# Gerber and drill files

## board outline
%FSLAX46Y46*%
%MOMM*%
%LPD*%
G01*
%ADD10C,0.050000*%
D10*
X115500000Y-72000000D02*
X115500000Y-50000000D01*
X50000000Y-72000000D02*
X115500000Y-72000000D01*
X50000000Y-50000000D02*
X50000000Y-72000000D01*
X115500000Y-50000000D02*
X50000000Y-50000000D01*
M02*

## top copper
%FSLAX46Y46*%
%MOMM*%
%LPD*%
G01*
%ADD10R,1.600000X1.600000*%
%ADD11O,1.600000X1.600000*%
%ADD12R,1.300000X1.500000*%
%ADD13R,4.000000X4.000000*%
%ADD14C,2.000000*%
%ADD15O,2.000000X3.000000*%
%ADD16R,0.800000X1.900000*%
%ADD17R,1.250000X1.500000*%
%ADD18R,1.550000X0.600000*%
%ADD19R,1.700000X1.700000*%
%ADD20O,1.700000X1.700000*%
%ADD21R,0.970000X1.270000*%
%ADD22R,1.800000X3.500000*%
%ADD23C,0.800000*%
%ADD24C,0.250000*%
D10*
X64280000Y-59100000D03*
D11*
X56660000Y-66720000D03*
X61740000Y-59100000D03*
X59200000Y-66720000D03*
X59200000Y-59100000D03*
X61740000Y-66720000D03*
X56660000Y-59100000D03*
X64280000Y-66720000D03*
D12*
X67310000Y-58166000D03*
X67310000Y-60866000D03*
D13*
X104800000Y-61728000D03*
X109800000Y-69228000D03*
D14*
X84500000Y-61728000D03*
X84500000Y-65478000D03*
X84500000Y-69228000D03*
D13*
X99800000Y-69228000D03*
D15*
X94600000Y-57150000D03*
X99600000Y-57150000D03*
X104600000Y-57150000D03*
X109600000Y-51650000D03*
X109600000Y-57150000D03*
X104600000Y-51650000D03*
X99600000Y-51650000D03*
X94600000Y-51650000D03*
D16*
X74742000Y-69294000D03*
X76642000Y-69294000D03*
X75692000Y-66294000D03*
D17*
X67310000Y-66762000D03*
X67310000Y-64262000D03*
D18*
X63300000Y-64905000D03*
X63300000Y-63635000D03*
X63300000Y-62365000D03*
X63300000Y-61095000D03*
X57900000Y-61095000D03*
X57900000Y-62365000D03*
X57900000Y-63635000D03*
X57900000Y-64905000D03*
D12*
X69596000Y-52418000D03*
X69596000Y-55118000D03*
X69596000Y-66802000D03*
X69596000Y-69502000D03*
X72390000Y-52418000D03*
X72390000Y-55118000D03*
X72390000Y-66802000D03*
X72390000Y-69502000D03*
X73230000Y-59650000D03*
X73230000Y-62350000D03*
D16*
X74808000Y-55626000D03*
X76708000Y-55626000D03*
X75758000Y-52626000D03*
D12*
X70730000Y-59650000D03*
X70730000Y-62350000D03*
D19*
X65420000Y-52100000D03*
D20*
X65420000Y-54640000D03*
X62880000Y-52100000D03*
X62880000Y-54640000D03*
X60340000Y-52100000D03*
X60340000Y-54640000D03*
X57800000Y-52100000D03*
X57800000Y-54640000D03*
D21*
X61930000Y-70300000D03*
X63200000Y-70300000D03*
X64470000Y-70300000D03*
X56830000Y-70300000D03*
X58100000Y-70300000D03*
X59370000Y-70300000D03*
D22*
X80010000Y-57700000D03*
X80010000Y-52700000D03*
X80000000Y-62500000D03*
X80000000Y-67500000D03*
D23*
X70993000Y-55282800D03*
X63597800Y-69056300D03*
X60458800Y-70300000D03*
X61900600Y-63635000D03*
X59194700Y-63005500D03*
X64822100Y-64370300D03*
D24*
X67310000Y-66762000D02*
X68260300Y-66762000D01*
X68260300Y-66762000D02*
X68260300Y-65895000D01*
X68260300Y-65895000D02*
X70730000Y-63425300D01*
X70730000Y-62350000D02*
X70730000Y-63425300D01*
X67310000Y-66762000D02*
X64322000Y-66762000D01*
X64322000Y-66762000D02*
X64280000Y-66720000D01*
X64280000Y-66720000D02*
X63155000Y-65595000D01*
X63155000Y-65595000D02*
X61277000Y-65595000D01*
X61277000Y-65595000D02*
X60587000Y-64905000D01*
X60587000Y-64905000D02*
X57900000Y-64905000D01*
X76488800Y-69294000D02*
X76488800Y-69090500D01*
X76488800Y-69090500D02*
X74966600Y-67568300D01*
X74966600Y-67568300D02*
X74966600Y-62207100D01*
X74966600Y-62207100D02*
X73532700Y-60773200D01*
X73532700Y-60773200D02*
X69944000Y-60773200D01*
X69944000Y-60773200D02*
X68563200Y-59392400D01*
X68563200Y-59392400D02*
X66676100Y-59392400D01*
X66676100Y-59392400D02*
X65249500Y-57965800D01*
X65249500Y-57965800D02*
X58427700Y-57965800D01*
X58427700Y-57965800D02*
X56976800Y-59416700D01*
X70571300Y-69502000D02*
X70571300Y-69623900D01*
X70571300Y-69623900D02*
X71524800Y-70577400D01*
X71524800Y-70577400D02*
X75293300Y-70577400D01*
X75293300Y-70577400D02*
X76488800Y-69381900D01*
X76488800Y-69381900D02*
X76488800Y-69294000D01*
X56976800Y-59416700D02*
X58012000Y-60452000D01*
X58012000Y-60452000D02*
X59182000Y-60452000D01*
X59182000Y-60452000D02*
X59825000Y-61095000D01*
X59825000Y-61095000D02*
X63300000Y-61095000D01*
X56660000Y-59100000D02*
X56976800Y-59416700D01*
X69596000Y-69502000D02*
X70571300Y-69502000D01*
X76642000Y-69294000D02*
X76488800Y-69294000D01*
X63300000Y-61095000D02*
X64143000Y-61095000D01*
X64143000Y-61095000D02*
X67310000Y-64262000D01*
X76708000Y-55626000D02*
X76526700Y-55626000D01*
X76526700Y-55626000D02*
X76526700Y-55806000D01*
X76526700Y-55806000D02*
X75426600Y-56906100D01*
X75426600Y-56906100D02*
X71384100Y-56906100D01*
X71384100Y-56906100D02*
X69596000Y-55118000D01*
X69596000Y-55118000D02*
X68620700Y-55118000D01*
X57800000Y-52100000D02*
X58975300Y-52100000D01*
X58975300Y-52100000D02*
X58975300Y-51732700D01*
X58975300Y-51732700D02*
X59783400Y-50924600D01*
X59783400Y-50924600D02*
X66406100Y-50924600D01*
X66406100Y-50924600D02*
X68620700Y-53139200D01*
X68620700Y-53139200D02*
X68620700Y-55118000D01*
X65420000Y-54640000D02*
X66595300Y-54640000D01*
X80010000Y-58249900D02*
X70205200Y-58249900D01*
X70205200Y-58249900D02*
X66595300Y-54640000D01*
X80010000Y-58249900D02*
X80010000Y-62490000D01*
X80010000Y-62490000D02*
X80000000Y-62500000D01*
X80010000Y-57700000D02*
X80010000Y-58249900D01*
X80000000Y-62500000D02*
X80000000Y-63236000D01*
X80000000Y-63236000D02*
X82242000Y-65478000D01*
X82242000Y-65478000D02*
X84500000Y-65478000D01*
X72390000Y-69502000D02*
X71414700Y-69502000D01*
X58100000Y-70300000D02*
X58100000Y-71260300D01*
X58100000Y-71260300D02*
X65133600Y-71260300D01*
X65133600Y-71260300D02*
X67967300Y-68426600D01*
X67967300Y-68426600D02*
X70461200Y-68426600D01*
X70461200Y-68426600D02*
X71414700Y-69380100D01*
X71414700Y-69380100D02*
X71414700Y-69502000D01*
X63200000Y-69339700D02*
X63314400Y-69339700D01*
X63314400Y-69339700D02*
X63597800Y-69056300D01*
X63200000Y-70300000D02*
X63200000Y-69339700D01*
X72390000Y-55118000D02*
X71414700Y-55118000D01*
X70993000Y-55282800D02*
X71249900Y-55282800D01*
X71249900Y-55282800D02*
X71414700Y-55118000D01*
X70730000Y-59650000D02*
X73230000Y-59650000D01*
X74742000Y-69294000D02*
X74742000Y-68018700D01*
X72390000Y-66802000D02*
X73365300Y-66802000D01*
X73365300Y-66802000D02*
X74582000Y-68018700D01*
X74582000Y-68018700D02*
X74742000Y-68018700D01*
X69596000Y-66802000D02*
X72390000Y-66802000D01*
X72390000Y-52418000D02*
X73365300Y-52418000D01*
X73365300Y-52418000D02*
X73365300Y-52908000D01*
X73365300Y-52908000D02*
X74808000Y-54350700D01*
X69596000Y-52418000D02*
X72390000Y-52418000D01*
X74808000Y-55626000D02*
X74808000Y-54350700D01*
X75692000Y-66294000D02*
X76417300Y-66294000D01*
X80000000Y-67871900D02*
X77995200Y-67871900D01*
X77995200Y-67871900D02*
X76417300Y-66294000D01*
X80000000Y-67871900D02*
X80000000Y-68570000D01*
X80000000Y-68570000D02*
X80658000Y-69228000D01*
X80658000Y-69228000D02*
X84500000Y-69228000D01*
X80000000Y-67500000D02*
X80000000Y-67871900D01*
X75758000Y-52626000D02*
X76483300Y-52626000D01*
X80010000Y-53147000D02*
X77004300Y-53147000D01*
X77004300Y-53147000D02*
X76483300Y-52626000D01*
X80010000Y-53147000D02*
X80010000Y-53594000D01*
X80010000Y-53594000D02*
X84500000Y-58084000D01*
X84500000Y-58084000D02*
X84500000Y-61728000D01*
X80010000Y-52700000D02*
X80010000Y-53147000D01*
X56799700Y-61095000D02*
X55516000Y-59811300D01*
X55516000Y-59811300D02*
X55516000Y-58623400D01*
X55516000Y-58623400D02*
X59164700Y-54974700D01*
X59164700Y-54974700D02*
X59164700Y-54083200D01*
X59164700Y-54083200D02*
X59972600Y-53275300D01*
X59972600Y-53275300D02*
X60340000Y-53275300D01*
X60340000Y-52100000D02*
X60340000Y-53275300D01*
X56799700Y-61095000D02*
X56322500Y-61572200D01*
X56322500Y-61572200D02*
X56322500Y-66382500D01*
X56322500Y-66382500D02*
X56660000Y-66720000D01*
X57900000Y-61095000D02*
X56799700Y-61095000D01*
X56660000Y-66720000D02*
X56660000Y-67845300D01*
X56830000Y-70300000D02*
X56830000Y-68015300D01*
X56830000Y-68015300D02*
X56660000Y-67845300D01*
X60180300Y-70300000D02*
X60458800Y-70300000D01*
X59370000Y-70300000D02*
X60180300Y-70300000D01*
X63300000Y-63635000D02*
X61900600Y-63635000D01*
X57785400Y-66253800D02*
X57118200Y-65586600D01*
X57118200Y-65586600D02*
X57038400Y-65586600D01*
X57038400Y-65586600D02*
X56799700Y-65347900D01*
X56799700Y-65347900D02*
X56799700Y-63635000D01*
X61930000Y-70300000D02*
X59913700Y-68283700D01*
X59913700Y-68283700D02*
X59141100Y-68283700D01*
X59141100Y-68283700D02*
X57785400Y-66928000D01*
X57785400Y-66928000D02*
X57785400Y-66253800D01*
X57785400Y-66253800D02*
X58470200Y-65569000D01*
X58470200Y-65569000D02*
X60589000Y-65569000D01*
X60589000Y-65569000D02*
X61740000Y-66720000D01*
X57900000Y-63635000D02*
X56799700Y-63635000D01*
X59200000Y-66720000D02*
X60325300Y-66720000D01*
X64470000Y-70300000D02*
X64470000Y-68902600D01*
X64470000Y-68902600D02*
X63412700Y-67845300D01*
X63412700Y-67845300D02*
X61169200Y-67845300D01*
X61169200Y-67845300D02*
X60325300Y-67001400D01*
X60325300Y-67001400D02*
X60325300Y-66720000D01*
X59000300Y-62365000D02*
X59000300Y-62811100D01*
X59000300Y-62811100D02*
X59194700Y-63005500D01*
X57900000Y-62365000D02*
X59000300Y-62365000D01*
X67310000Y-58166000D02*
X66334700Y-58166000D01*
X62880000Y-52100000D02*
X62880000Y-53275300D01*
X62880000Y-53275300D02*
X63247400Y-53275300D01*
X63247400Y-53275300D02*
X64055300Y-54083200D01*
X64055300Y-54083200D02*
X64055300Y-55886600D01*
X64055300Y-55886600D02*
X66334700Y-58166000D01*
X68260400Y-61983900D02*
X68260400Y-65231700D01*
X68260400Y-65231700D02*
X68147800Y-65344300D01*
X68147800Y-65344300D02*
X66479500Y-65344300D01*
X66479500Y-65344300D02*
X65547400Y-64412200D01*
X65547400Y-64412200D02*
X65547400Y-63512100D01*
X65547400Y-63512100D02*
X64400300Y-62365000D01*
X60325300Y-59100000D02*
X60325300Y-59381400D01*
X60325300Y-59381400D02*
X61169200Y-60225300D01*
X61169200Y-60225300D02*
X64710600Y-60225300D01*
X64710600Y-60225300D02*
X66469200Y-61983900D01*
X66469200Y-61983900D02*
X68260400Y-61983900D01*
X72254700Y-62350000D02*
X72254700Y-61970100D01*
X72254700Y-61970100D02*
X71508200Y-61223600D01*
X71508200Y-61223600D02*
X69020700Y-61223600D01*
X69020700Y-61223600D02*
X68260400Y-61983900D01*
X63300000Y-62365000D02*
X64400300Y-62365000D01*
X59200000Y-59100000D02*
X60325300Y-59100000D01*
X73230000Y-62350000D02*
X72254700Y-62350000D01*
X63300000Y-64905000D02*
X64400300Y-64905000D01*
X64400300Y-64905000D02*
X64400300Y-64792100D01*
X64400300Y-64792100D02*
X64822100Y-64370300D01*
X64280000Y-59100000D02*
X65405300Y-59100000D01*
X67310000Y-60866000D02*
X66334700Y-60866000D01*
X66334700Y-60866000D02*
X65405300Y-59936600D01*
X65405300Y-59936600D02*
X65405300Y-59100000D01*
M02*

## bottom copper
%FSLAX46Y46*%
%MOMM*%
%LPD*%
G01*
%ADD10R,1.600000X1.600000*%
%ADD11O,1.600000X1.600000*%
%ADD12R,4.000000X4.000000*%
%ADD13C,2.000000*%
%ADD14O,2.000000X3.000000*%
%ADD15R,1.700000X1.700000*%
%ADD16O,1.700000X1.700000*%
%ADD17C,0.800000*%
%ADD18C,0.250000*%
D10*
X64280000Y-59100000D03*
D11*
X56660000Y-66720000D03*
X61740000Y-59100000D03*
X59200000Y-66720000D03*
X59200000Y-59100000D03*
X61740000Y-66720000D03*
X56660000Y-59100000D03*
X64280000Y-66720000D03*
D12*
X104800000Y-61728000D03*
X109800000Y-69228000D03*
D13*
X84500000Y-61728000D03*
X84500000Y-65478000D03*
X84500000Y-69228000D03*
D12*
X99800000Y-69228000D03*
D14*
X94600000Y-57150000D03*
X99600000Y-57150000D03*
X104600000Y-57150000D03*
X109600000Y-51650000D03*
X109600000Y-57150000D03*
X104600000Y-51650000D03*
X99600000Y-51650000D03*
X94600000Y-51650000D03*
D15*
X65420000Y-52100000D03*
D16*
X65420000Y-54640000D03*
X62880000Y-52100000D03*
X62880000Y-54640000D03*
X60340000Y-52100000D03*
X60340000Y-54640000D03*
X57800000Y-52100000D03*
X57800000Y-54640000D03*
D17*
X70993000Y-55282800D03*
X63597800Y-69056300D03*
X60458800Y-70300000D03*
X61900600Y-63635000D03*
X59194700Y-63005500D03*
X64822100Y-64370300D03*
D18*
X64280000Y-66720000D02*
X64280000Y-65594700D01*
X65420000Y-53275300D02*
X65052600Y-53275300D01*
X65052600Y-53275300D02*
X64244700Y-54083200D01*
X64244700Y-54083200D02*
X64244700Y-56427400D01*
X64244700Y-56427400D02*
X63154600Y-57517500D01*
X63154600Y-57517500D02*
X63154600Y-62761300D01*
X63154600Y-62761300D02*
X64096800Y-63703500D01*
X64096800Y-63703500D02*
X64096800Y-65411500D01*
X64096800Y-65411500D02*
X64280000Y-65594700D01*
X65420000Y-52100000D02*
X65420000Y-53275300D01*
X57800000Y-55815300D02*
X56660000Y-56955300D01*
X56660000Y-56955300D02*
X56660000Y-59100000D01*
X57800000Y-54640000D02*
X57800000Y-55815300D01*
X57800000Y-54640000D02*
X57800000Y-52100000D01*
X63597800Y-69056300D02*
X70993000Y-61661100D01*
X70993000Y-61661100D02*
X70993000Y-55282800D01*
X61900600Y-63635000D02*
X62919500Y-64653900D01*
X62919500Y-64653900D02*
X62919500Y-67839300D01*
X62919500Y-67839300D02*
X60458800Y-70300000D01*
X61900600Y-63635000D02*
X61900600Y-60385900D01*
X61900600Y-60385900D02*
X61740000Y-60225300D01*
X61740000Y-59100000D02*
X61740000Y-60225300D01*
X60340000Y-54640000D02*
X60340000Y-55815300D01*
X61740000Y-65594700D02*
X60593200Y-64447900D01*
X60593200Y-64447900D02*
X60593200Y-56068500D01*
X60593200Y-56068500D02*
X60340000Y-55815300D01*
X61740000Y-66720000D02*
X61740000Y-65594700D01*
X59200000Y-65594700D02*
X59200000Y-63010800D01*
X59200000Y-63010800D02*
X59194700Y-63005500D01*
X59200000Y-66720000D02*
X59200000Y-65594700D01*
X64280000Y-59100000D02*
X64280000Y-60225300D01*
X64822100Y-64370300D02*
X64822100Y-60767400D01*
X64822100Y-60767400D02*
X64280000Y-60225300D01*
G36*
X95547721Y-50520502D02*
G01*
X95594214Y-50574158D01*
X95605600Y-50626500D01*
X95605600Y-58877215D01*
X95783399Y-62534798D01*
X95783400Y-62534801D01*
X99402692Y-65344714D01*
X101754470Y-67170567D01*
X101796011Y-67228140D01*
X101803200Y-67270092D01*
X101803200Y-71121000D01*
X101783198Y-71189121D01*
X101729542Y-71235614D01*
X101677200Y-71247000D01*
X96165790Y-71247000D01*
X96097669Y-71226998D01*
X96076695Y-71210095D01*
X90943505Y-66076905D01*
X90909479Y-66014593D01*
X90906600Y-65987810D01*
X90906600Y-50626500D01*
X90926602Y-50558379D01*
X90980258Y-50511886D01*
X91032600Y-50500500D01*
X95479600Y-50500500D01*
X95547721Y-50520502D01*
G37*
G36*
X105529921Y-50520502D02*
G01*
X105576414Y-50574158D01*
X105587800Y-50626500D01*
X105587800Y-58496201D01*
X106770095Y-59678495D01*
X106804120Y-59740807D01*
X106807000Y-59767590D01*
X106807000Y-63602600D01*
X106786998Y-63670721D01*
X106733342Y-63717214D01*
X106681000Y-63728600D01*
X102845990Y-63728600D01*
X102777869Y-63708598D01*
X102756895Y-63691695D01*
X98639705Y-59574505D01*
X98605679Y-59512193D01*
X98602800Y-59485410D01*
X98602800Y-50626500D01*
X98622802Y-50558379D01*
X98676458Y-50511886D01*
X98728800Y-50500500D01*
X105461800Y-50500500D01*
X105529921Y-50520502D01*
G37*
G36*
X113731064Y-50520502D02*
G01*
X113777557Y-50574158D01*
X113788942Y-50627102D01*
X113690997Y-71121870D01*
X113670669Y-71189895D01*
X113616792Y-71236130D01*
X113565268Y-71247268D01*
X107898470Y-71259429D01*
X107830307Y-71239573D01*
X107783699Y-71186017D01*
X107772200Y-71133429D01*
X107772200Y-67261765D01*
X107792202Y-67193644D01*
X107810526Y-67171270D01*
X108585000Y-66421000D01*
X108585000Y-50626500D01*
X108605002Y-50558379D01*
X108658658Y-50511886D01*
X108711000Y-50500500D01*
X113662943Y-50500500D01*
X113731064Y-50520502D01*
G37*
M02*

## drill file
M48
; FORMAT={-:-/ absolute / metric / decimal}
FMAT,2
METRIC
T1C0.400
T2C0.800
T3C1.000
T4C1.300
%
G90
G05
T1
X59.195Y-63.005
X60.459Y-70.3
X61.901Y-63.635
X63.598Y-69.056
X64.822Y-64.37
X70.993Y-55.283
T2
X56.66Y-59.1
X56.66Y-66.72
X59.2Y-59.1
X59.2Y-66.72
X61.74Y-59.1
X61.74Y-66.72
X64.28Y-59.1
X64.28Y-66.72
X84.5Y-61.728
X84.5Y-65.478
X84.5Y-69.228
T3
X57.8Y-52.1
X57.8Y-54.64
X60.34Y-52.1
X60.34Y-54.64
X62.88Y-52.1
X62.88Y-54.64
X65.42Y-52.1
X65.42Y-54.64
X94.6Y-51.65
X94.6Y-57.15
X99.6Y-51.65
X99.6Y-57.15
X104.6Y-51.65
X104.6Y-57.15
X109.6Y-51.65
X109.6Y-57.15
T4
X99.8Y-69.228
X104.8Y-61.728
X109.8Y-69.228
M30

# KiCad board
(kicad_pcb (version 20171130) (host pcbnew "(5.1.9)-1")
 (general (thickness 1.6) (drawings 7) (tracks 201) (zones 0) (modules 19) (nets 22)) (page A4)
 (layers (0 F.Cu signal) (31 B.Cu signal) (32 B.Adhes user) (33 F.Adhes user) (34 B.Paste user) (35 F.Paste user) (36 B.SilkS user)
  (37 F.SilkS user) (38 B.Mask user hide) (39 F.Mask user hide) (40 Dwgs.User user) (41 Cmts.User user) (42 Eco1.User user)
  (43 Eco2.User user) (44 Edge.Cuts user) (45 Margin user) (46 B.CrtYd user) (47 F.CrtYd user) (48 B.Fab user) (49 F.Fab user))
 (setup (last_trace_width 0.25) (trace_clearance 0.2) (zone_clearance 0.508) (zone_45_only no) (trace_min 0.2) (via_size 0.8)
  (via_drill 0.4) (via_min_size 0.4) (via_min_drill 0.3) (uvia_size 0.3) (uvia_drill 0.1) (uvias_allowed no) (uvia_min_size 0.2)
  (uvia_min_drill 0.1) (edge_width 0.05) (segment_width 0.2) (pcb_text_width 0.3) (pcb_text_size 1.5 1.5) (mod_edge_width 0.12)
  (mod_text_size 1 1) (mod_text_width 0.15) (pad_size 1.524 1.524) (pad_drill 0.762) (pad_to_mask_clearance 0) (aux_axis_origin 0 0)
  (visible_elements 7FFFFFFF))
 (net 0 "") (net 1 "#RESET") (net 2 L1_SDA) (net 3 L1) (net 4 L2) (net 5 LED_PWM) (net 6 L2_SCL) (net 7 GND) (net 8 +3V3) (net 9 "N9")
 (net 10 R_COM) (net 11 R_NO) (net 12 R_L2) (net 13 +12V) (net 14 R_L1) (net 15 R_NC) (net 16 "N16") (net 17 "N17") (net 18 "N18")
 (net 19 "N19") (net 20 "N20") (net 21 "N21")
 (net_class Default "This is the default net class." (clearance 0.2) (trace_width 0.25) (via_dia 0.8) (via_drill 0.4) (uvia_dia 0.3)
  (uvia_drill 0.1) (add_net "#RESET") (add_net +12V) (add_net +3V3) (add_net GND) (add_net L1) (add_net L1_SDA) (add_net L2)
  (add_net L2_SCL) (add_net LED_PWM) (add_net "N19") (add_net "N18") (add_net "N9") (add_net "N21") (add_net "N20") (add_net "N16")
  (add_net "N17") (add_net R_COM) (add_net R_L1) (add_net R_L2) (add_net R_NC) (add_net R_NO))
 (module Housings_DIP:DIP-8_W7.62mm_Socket (layer F.Cu) (at 64.28 59.1 270)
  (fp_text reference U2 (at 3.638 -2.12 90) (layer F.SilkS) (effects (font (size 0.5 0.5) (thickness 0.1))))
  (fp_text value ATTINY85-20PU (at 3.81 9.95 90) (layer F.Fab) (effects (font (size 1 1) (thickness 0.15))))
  (pad 1 thru_hole rect (at 0 0 270) (size 1.6 1.6) (drill 0.8) (layers *.Cu *.Mask) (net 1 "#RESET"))
  (pad 5 thru_hole oval (at 7.62 7.62 270) (size 1.6 1.6) (drill 0.8) (layers *.Cu *.Mask) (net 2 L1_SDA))
  (pad 2 thru_hole oval (at 0 2.54 270) (size 1.6 1.6) (drill 0.8) (layers *.Cu *.Mask) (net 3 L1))
  (pad 6 thru_hole oval (at 7.62 5.08 270) (size 1.6 1.6) (drill 0.8) (layers *.Cu *.Mask) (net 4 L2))
  (pad 3 thru_hole oval (at 0 5.08 270) (size 1.6 1.6) (drill 0.8) (layers *.Cu *.Mask) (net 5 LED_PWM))
  (pad 7 thru_hole oval (at 7.62 2.54 270) (size 1.6 1.6) (drill 0.8) (layers *.Cu *.Mask) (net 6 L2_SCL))
  (pad 4 thru_hole oval (at 0 7.62 270) (size 1.6 1.6) (drill 0.8) (layers *.Cu *.Mask) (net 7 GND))
  (pad 8 thru_hole oval (at 7.62 0 270) (size 1.6 1.6) (drill 0.8) (layers *.Cu *.Mask) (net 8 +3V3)))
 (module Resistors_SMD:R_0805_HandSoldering (layer F.Cu) (at 67.31 59.516 270)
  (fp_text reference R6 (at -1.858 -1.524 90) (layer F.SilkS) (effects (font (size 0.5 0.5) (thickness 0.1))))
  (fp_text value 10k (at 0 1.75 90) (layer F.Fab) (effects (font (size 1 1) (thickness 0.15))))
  (pad 1 smd rect (at -1.35 0 270) (size 1.5 1.3) (layers F.Cu F.Paste F.Mask) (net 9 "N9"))
  (pad 2 smd rect (at 1.35 0 270) (size 1.5 1.3) (layers F.Cu F.Paste F.Mask) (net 1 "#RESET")))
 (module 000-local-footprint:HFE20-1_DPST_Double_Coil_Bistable (layer F.Cu) (at 84.5 65.478)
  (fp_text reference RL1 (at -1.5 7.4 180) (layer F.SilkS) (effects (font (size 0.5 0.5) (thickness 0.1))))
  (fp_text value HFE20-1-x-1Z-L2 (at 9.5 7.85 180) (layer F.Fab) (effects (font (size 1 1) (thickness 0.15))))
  (pad 3 thru_hole rect (at 20.3 -3.75) (size 4 4) (drill 1.3) (layers *.Cu *.Mask) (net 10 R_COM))
  (pad 4 thru_hole rect (at 25.3 3.75) (size 4 4) (drill 1.3) (layers *.Cu *.Mask) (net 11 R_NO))
  (pad 2 thru_hole circle (at 0 -3.75) (size 2 2) (drill 0.8) (layers *.Cu *.Mask) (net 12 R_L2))
  (pad 5 thru_hole circle (at 0 0) (size 2 2) (drill 0.8) (layers *.Cu *.Mask) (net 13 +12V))
  (pad 1 thru_hole circle (at 0 3.75) (size 2 2) (drill 0.8) (layers *.Cu *.Mask) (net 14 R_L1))
  (pad 6 thru_hole rect (at 15.3 3.75) (size 4 4) (drill 1.3) (layers *.Cu *.Mask) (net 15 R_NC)))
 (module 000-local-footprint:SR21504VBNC (layer F.Cu) (at 109.6 57.15 180)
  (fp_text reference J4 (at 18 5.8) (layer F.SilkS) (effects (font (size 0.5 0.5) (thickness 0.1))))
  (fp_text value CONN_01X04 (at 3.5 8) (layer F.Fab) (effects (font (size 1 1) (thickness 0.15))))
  (pad 4 thru_hole oval (at 15 0 180) (size 2 3) (drill 1) (layers *.Cu *.Mask) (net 15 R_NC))
  (pad 3 thru_hole oval (at 10 0 180) (size 2 3) (drill 1) (layers *.Cu *.Mask) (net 10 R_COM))
  (pad 2 thru_hole oval (at 5 0 180) (size 2 3) (drill 1) (layers *.Cu *.Mask) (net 10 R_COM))
  (pad 1 thru_hole oval (at 0 5.5 180) (size 2 3) (drill 1) (layers *.Cu *.Mask) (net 11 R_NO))
  (pad 1 thru_hole oval (at 0 0 180) (size 2 3) (drill 1) (layers *.Cu *.Mask) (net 11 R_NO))
  (pad 2 thru_hole oval (at 5 5.5 180) (size 2 3) (drill 1) (layers *.Cu *.Mask) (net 10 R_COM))
  (pad 3 thru_hole oval (at 10 5.5 180) (size 2 3) (drill 1) (layers *.Cu *.Mask) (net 10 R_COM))
  (pad 4 thru_hole oval (at 15 5.5 180) (size 2 3) (drill 1) (layers *.Cu *.Mask) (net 15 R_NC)))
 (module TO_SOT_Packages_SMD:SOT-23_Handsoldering (layer F.Cu) (at 75.692 67.794 90)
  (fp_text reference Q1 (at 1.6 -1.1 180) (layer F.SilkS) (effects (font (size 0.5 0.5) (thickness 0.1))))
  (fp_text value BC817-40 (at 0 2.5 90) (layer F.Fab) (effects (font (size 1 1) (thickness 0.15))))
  (pad 1 smd rect (at -1.5 -0.95 90) (size 1.9 0.8) (layers F.Cu F.Paste F.Mask) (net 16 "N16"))
  (pad 2 smd rect (at -1.5 0.95 90) (size 1.9 0.8) (layers F.Cu F.Paste F.Mask) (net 7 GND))
  (pad 3 smd rect (at 1.5 0 90) (size 1.9 0.8) (layers F.Cu F.Paste F.Mask) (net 14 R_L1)))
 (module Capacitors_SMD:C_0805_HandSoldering (layer F.Cu) (at 67.31 65.512 90)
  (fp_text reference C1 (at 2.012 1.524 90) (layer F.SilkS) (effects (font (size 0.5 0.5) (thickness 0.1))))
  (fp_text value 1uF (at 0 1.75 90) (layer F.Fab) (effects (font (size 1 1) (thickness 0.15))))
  (pad 1 smd rect (at -1.25 0 90) (size 1.5 1.25) (layers F.Cu F.Paste F.Mask) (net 8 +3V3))
  (pad 2 smd rect (at 1.25 0 90) (size 1.5 1.25) (layers F.Cu F.Paste F.Mask) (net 7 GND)))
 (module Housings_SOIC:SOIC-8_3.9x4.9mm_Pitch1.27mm (layer F.Cu) (at 60.6 63 180)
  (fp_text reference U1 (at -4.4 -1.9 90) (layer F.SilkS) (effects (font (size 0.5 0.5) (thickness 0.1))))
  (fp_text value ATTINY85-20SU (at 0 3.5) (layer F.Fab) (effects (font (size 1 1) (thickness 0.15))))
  (pad 1 smd rect (at -2.7 -1.905 180) (size 1.55 0.6) (layers F.Cu F.Paste F.Mask) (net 1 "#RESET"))
  (pad 2 smd rect (at -2.7 -0.635 180) (size 1.55 0.6) (layers F.Cu F.Paste F.Mask) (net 3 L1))
  (pad 3 smd rect (at -2.7 0.635 180) (size 1.55 0.6) (layers F.Cu F.Paste F.Mask) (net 5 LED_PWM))
  (pad 4 smd rect (at -2.7 1.905 180) (size 1.55 0.6) (layers F.Cu F.Paste F.Mask) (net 7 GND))
  (pad 5 smd rect (at 2.7 1.905 180) (size 1.55 0.6) (layers F.Cu F.Paste F.Mask) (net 2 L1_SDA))
  (pad 6 smd rect (at 2.7 0.635 180) (size 1.55 0.6) (layers F.Cu F.Paste F.Mask) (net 4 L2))
  (pad 7 smd rect (at 2.7 -0.635 180) (size 1.55 0.6) (layers F.Cu F.Paste F.Mask) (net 6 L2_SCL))
  (pad 8 smd rect (at 2.7 -1.905 180) (size 1.55 0.6) (layers F.Cu F.Paste F.Mask) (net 8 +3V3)))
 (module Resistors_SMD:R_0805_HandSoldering (layer F.Cu) (at 69.596 53.768 270)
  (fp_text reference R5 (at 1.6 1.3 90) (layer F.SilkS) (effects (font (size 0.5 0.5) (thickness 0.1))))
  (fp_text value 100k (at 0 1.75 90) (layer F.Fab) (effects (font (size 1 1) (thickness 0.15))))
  (pad 1 smd rect (at -1.35 0 270) (size 1.5 1.3) (layers F.Cu F.Paste F.Mask) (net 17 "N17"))
  (pad 2 smd rect (at 1.35 0 270) (size 1.5 1.3) (layers F.Cu F.Paste F.Mask) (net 7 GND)))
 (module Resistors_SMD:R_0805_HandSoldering (layer F.Cu) (at 69.596 68.152 270)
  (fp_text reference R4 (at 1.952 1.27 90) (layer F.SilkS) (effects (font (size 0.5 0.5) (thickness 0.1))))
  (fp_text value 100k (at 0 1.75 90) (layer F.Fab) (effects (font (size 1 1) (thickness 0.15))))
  (pad 1 smd rect (at -1.35 0 270) (size 1.5 1.3) (layers F.Cu F.Paste F.Mask) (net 16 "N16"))
  (pad 2 smd rect (at 1.35 0 270) (size 1.5 1.3) (layers F.Cu F.Paste F.Mask) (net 7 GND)))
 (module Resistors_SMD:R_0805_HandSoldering (layer F.Cu) (at 72.39 53.768 270)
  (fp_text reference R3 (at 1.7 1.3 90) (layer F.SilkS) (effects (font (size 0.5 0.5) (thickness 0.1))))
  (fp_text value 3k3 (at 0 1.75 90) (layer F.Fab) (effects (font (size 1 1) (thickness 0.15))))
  (pad 1 smd rect (at -1.35 0 270) (size 1.5 1.3) (layers F.Cu F.Paste F.Mask) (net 17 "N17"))
  (pad 2 smd rect (at 1.35 0 270) (size 1.5 1.3) (layers F.Cu F.Paste F.Mask) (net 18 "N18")))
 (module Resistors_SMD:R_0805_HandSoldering (layer F.Cu) (at 72.39 68.152 270)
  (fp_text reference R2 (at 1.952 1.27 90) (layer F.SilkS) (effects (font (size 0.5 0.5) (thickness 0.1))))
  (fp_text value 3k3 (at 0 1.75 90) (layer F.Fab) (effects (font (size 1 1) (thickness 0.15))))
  (pad 1 smd rect (at -1.35 0 270) (size 1.5 1.3) (layers F.Cu F.Paste F.Mask) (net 16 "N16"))
  (pad 2 smd rect (at 1.35 0 270) (size 1.5 1.3) (layers F.Cu F.Paste F.Mask) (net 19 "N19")))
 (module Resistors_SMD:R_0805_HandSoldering (layer F.Cu) (at 73.23 61 270)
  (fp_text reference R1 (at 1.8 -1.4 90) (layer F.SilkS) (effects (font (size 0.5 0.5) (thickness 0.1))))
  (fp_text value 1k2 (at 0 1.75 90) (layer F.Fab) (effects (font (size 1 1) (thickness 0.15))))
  (pad 1 smd rect (at -1.35 0 270) (size 1.5 1.3) (layers F.Cu F.Paste F.Mask) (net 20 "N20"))
  (pad 2 smd rect (at 1.35 0 270) (size 1.5 1.3) (layers F.Cu F.Paste F.Mask) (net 5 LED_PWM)))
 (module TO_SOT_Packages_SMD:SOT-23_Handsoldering (layer F.Cu) (at 75.758 54.126 90)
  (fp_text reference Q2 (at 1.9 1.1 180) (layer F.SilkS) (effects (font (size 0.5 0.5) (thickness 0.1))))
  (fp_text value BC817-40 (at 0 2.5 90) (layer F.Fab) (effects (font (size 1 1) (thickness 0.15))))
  (pad 1 smd rect (at -1.5 -0.95 90) (size 1.9 0.8) (layers F.Cu F.Paste F.Mask) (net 17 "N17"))
  (pad 2 smd rect (at -1.5 0.95 90) (size 1.9 0.8) (layers F.Cu F.Paste F.Mask) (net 7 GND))
  (pad 3 smd rect (at 1.5 0 90) (size 1.9 0.8) (layers F.Cu F.Paste F.Mask) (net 12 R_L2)))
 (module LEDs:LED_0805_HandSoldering (layer F.Cu) (at 70.73 61 270)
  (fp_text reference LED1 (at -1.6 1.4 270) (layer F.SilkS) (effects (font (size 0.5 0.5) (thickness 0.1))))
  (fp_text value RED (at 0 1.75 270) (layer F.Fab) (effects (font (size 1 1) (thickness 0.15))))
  (pad 1 smd rect (at -1.35 0 270) (size 1.5 1.3) (layers F.Cu F.Paste F.Mask) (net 20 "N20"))
  (pad 2 smd rect (at 1.35 0 270) (size 1.5 1.3) (layers F.Cu F.Paste F.Mask) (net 8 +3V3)))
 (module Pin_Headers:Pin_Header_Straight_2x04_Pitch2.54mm (layer F.Cu) (at 65.42 52.1 270)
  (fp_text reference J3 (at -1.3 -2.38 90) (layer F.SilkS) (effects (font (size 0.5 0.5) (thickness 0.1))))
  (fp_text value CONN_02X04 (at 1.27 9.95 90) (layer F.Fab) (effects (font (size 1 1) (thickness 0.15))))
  (pad 1 thru_hole rect (at 0 0 270) (size 1.7 1.7) (drill 1) (layers *.Cu *.Mask) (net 8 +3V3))
  (pad 2 thru_hole oval (at 2.54 0 270) (size 1.7 1.7) (drill 1) (layers *.Cu *.Mask) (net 13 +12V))
  (pad 3 thru_hole oval (at 0 2.54 270) (size 1.7 1.7) (drill 1) (layers *.Cu *.Mask) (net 9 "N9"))
  (pad 4 thru_hole oval (at 2.54 2.54 270) (size 1.7 1.7) (drill 1) (layers *.Cu *.Mask) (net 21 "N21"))
  (pad 5 thru_hole oval (at 0 5.08 270) (size 1.7 1.7) (drill 1) (layers *.Cu *.Mask) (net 2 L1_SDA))
  (pad 6 thru_hole oval (at 2.54 5.08 270) (size 1.7 1.7) (drill 1) (layers *.Cu *.Mask) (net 6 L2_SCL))
  (pad 7 thru_hole oval (at 0 7.62 270) (size 1.7 1.7) (drill 1) (layers *.Cu *.Mask) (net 7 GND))
  (pad 8 thru_hole oval (at 2.54 7.62 270) (size 1.7 1.7) (drill 1) (layers *.Cu *.Mask) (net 7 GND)))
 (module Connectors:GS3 (layer F.Cu) (at 63.2 70.3 90)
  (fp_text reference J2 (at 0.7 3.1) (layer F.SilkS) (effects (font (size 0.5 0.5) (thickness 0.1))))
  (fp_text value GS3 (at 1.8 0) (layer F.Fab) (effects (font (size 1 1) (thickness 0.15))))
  (pad 1 smd rect (at 0 -1.27 90) (size 1.27 0.97) (layers F.Cu F.Paste F.Mask) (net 6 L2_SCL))
  (pad 2 smd rect (at 0 0 90) (size 1.27 0.97) (layers F.Cu F.Paste F.Mask) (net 18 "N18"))
  (pad 3 smd rect (at 0 1.27 90) (size 1.27 0.97) (layers F.Cu F.Paste F.Mask) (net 4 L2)))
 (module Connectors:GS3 (layer F.Cu) (at 58.1 70.3 90)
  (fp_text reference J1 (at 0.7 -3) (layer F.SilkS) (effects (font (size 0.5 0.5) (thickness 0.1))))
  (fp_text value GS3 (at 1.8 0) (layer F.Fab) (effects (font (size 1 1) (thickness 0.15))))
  (pad 1 smd rect (at 0 -1.27 90) (size 1.27 0.97) (layers F.Cu F.Paste F.Mask) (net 2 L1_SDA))
  (pad 2 smd rect (at 0 0 90) (size 1.27 0.97) (layers F.Cu F.Paste F.Mask) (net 19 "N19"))
  (pad 3 smd rect (at 0 1.27 90) (size 1.27 0.97) (layers F.Cu F.Paste F.Mask) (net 3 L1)))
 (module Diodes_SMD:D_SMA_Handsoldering (layer F.Cu) (at 80.01 55.2 90)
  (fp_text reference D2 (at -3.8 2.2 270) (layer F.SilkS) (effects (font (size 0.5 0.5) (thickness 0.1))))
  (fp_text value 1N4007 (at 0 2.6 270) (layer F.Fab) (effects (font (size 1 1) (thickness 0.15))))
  (pad 1 smd rect (at -2.5 0 90) (size 3.5 1.8) (layers F.Cu F.Paste F.Mask) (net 13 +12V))
  (pad 2 smd rect (at 2.5 0 90) (size 3.5 1.8) (layers F.Cu F.Paste F.Mask) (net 12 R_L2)))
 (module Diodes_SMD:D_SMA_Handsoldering (layer F.Cu) (at 80 65 270)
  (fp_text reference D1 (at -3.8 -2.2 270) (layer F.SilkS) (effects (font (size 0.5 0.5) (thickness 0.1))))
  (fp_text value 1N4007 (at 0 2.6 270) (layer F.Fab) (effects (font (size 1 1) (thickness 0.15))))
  (pad 1 smd rect (at -2.5 0 270) (size 3.5 1.8) (layers F.Cu F.Paste F.Mask) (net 13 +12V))
  (pad 2 smd rect (at 2.5 0 270) (size 3.5 1.8) (layers F.Cu F.Paste F.Mask) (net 14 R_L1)))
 (gr_line (start 115.5 72) (end 115.5 50) (layer Edge.Cuts) (width 0.05))
 (gr_line (start 50 72) (end 115.5 72) (layer Edge.Cuts) (width 0.05))
 (gr_line (start 50 50) (end 50 72) (layer Edge.Cuts) (width 0.05))
 (gr_line (start 115.5 50) (end 50 50) (layer Edge.Cuts) (width 0.05))
 (segment (start 64.28 66.72) (end 64.28 65.5947) (width 0.25) (layer B.Cu) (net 8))
 (segment (start 65.42 53.2753) (end 65.0526 53.2753) (width 0.25) (layer B.Cu) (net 8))
 (segment (start 65.0526 53.2753) (end 64.2447 54.0832) (width 0.25) (layer B.Cu) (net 8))
 (segment (start 64.2447 54.0832) (end 64.2447 56.4274) (width 0.25) (layer B.Cu) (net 8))
 (segment (start 64.2447 56.4274) (end 63.1546 57.5175) (width 0.25) (layer B.Cu) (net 8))
 (segment (start 63.1546 57.5175) (end 63.1546 62.7613) (width 0.25) (layer B.Cu) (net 8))
 (segment (start 63.1546 62.7613) (end 64.0968 63.7035) (width 0.25) (layer B.Cu) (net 8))
 (segment (start 64.0968 63.7035) (end 64.0968 65.4115) (width 0.25) (layer B.Cu) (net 8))
 (segment (start 64.0968 65.4115) (end 64.28 65.5947) (width 0.25) (layer B.Cu) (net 8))
 (segment (start 67.31 66.762) (end 68.2603 66.762) (width 0.25) (layer F.Cu) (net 8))
 (segment (start 68.2603 66.762) (end 68.2603 65.895) (width 0.25) (layer F.Cu) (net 8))
 (segment (start 68.2603 65.895) (end 70.73 63.4253) (width 0.25) (layer F.Cu) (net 8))
 (segment (start 70.73 62.35) (end 70.73 63.4253) (width 0.25) (layer F.Cu) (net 8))
 (segment (start 67.31 66.762) (end 64.322 66.762) (width 0.25) (layer F.Cu) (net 8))
 (segment (start 64.322 66.762) (end 64.28 66.72) (width 0.25) (layer F.Cu) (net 8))
 (segment (start 65.42 52.1) (end 65.42 53.2753) (width 0.25) (layer B.Cu) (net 8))
 (segment (start 64.28 66.72) (end 63.155 65.595) (width 0.25) (layer F.Cu) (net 8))
 (segment (start 63.155 65.595) (end 61.277 65.595) (width 0.25) (layer F.Cu) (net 8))
 (segment (start 61.277 65.595) (end 60.587 64.905) (width 0.25) (layer F.Cu) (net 8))
 (segment (start 60.587 64.905) (end 57.9 64.905) (width 0.25) (layer F.Cu) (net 8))
 (segment (start 76.4888 69.294) (end 76.4888 69.0905) (width 0.25) (layer F.Cu) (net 7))
 (segment (start 76.4888 69.0905) (end 74.9666 67.5683) (width 0.25) (layer F.Cu) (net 7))
 (segment (start 74.9666 67.5683) (end 74.9666 62.2071) (width 0.25) (layer F.Cu) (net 7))
 (segment (start 74.9666 62.2071) (end 73.5327 60.7732) (width 0.25) (layer F.Cu) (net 7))
 (segment (start 73.5327 60.7732) (end 69.944 60.7732) (width 0.25) (layer F.Cu) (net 7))
 (segment (start 69.944 60.7732) (end 68.5632 59.3924) (width 0.25) (layer F.Cu) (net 7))
 (segment (start 68.5632 59.3924) (end 66.6761 59.3924) (width 0.25) (layer F.Cu) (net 7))
 (segment (start 66.6761 59.3924) (end 65.2495 57.9658) (width 0.25) (layer F.Cu) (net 7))
 (segment (start 65.2495 57.9658) (end 58.4277 57.9658) (width 0.25) (layer F.Cu) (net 7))
 (segment (start 58.4277 57.9658) (end 56.9768 59.4167) (width 0.25) (layer F.Cu) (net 7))
 (segment (start 70.5713 69.502) (end 70.5713 69.6239) (width 0.25) (layer F.Cu) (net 7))
 (segment (start 70.5713 69.6239) (end 71.5248 70.5774) (width 0.25) (layer F.Cu) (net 7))
 (segment (start 71.5248 70.5774) (end 75.2933 70.5774) (width 0.25) (layer F.Cu) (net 7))
 (segment (start 75.2933 70.5774) (end 76.4888 69.3819) (width 0.25) (layer F.Cu) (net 7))
 (segment (start 76.4888 69.3819) (end 76.4888 69.294) (width 0.25) (layer F.Cu) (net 7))
 (segment (start 56.9768 59.4167) (end 58.012 60.452) (width 0.25) (layer F.Cu) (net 7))
 (segment (start 58.012 60.452) (end 59.182 60.452) (width 0.25) (layer F.Cu) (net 7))
 (segment (start 59.182 60.452) (end 59.825 61.095) (width 0.25) (layer F.Cu) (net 7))
 (segment (start 59.825 61.095) (end 63.3 61.095) (width 0.25) (layer F.Cu) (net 7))
 (segment (start 56.66 59.1) (end 56.9768 59.4167) (width 0.25) (layer F.Cu) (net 7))
 (segment (start 69.596 69.502) (end 70.5713 69.502) (width 0.25) (layer F.Cu) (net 7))
 (segment (start 76.642 69.294) (end 76.4888 69.294) (width 0.25) (layer F.Cu) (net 7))
 (segment (start 63.3 61.095) (end 64.143 61.095) (width 0.25) (layer F.Cu) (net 7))
 (segment (start 64.143 61.095) (end 67.31 64.262) (width 0.25) (layer F.Cu) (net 7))
 (segment (start 76.708 55.626) (end 76.5267 55.626) (width 0.25) (layer F.Cu) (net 7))
 (segment (start 76.5267 55.626) (end 76.5267 55.806) (width 0.25) (layer F.Cu) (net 7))
 (segment (start 76.5267 55.806) (end 75.4266 56.9061) (width 0.25) (layer F.Cu) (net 7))
 (segment (start 75.4266 56.9061) (end 71.3841 56.9061) (width 0.25) (layer F.Cu) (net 7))
 (segment (start 71.3841 56.9061) (end 69.596 55.118) (width 0.25) (layer F.Cu) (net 7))
 (segment (start 69.596 55.118) (end 68.6207 55.118) (width 0.25) (layer F.Cu) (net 7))
 (segment (start 57.8 52.1) (end 58.9753 52.1) (width 0.25) (layer F.Cu) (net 7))
 (segment (start 58.9753 52.1) (end 58.9753 51.7327) (width 0.25) (layer F.Cu) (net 7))
 (segment (start 58.9753 51.7327) (end 59.7834 50.9246) (width 0.25) (layer F.Cu) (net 7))
 (segment (start 59.7834 50.9246) (end 66.4061 50.9246) (width 0.25) (layer F.Cu) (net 7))
 (segment (start 66.4061 50.9246) (end 68.6207 53.1392) (width 0.25) (layer F.Cu) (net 7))
 (segment (start 68.6207 53.1392) (end 68.6207 55.118) (width 0.25) (layer F.Cu) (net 7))
 (segment (start 57.8 55.8153) (end 56.66 56.9553) (width 0.25) (layer B.Cu) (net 7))
 (segment (start 56.66 56.9553) (end 56.66 59.1) (width 0.25) (layer B.Cu) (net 7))
 (segment (start 57.8 54.64) (end 57.8 55.8153) (width 0.25) (layer B.Cu) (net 7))
 (segment (start 57.8 54.64) (end 57.8 52.1) (width 0.25) (layer B.Cu) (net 7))
 (segment (start 65.42 54.64) (end 66.5953 54.64) (width 0.25) (layer F.Cu) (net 13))
 (segment (start 80.01 58.2499) (end 70.2052 58.2499) (width 0.25) (layer F.Cu) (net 13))
 (segment (start 70.2052 58.2499) (end 66.5953 54.64) (width 0.25) (layer F.Cu) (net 13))
 (segment (start 80.01 58.2499) (end 80.01 62.49) (width 0.25) (layer F.Cu) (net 13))
 (segment (start 80.01 62.49) (end 80 62.5) (width 0.25) (layer F.Cu) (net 13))
 (segment (start 80.01 57.7) (end 80.01 58.2499) (width 0.25) (layer F.Cu) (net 13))
 (segment (start 80 62.5) (end 80 63.236) (width 0.25) (layer F.Cu) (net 13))
 (segment (start 80 63.236) (end 82.242 65.478) (width 0.25) (layer F.Cu) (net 13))
 (segment (start 82.242 65.478) (end 84.5 65.478) (width 0.25) (layer F.Cu) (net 13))
 (segment (start 72.39 69.502) (end 71.4147 69.502) (width 0.25) (layer F.Cu) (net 19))
 (segment (start 58.1 70.3) (end 58.1 71.2603) (width 0.25) (layer F.Cu) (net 19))
 (segment (start 58.1 71.2603) (end 65.1336 71.2603) (width 0.25) (layer F.Cu) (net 19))
 (segment (start 65.1336 71.2603) (end 67.9673 68.4266) (width 0.25) (layer F.Cu) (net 19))
 (segment (start 67.9673 68.4266) (end 70.4612 68.4266) (width 0.25) (layer F.Cu) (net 19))
 (segment (start 70.4612 68.4266) (end 71.4147 69.3801) (width 0.25) (layer F.Cu) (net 19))
 (segment (start 71.4147 69.3801) (end 71.4147 69.502) (width 0.25) (layer F.Cu) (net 19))
 (segment (start 63.2 69.3397) (end 63.3144 69.3397) (width 0.25) (layer F.Cu) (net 18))
 (segment (start 63.3144 69.3397) (end 63.5978 69.0563) (width 0.25) (layer F.Cu) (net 18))
 (segment (start 63.5978 69.0563) (end 70.993 61.6611) (width 0.25) (layer B.Cu) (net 18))
 (segment (start 70.993 61.6611) (end 70.993 55.2828) (width 0.25) (layer B.Cu) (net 18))
 (segment (start 63.2 70.3) (end 63.2 69.3397) (width 0.25) (layer F.Cu) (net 18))
 (segment (start 72.39 55.118) (end 71.4147 55.118) (width 0.25) (layer F.Cu) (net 18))
 (segment (start 70.993 55.2828) (end 71.2499 55.2828) (width 0.25) (layer F.Cu) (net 18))
 (segment (start 71.2499 55.2828) (end 71.4147 55.118) (width 0.25) (layer F.Cu) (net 18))
 (via (at 70.993 55.2828) (size 0.8) (layers F.Cu B.Cu) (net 18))
 (via (at 63.5978 69.0563) (size 0.8) (layers F.Cu B.Cu) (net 18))
 (segment (start 70.73 59.65) (end 73.23 59.65) (width 0.25) (layer F.Cu) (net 20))
 (segment (start 74.742 69.294) (end 74.742 68.0187) (width 0.25) (layer F.Cu) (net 16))
 (segment (start 72.39 66.802) (end 73.3653 66.802) (width 0.25) (layer F.Cu) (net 16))
 (segment (start 73.3653 66.802) (end 74.582 68.0187) (width 0.25) (layer F.Cu) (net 16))
 (segment (start 74.582 68.0187) (end 74.742 68.0187) (width 0.25) (layer F.Cu) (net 16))
 (segment (start 69.596 66.802) (end 72.39 66.802) (width 0.25) (layer F.Cu) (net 16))
 (segment (start 72.39 52.418) (end 73.3653 52.418) (width 0.25) (layer F.Cu) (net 17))
 (segment (start 73.3653 52.418) (end 73.3653 52.908) (width 0.25) (layer F.Cu) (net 17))
 (segment (start 73.3653 52.908) (end 74.808 54.3507) (width 0.25) (layer F.Cu) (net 17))
 (segment (start 69.596 52.418) (end 72.39 52.418) (width 0.25) (layer F.Cu) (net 17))
 (segment (start 74.808 55.626) (end 74.808 54.3507) (width 0.25) (layer F.Cu) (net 17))
 (segment (start 75.692 66.294) (end 76.4173 66.294) (width 0.25) (layer F.Cu) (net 14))
 (segment (start 80 67.8719) (end 77.9952 67.8719) (width 0.25) (layer F.Cu) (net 14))
 (segment (start 77.9952 67.8719) (end 76.4173 66.294) (width 0.25) (layer F.Cu) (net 14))
 (segment (start 80 67.8719) (end 80 68.57) (width 0.25) (layer F.Cu) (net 14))
 (segment (start 80 68.57) (end 80.658 69.228) (width 0.25) (layer F.Cu) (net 14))
 (segment (start 80.658 69.228) (end 84.5 69.228) (width 0.25) (layer F.Cu) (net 14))
 (segment (start 80 67.5) (end 80 67.8719) (width 0.25) (layer F.Cu) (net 14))
 (segment (start 75.758 52.626) (end 76.4833 52.626) (width 0.25) (layer F.Cu) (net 12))
 (segment (start 80.01 53.147) (end 77.0043 53.147) (width 0.25) (layer F.Cu) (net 12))
 (segment (start 77.0043 53.147) (end 76.4833 52.626) (width 0.25) (layer F.Cu) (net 12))
 (segment (start 80.01 53.147) (end 80.01 53.594) (width 0.25) (layer F.Cu) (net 12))
 (segment (start 80.01 53.594) (end 84.5 58.084) (width 0.25) (layer F.Cu) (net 12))
 (segment (start 84.5 58.084) (end 84.5 61.728) (width 0.25) (layer F.Cu) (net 12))
 (segment (start 80.01 52.7) (end 80.01 53.147) (width 0.25) (layer F.Cu) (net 12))
 (segment (start 56.7997 61.095) (end 55.516 59.8113) (width 0.25) (layer F.Cu) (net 2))
 (segment (start 55.516 59.8113) (end 55.516 58.6234) (width 0.25) (layer F.Cu) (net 2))
 (segment (start 55.516 58.6234) (end 59.1647 54.9747) (width 0.25) (layer F.Cu) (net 2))
 (segment (start 59.1647 54.9747) (end 59.1647 54.0832) (width 0.25) (layer F.Cu) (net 2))
 (segment (start 59.1647 54.0832) (end 59.9726 53.2753) (width 0.25) (layer F.Cu) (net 2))
 (segment (start 59.9726 53.2753) (end 60.34 53.2753) (width 0.25) (layer F.Cu) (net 2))
 (segment (start 60.34 52.1) (end 60.34 53.2753) (width 0.25) (layer F.Cu) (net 2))
 (segment (start 56.7997 61.095) (end 56.3225 61.5722) (width 0.25) (layer F.Cu) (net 2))
 (segment (start 56.3225 61.5722) (end 56.3225 66.3825) (width 0.25) (layer F.Cu) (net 2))
 (segment (start 56.3225 66.3825) (end 56.66 66.72) (width 0.25) (layer F.Cu) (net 2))
 (segment (start 57.9 61.095) (end 56.7997 61.095) (width 0.25) (layer F.Cu) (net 2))
 (segment (start 56.66 66.72) (end 56.66 67.8453) (width 0.25) (layer F.Cu) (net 2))
 (segment (start 56.83 70.3) (end 56.83 68.0153) (width 0.25) (layer F.Cu) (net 2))
 (segment (start 56.83 68.0153) (end 56.66 67.8453) (width 0.25) (layer F.Cu) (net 2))
 (segment (start 60.1803 70.3) (end 60.4588 70.3) (width 0.25) (layer F.Cu) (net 3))
 (segment (start 61.9006 63.635) (end 62.9195 64.6539) (width 0.25) (layer B.Cu) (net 3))
 (segment (start 62.9195 64.6539) (end 62.9195 67.8393) (width 0.25) (layer B.Cu) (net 3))
 (segment (start 62.9195 67.8393) (end 60.4588 70.3) (width 0.25) (layer B.Cu) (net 3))
 (segment (start 59.37 70.3) (end 60.1803 70.3) (width 0.25) (layer F.Cu) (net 3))
 (segment (start 61.9006 63.635) (end 61.9006 60.3859) (width 0.25) (layer B.Cu) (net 3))
 (segment (start 61.9006 60.3859) (end 61.74 60.2253) (width 0.25) (layer B.Cu) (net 3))
 (segment (start 63.3 63.635) (end 61.9006 63.635) (width 0.25) (layer F.Cu) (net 3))
 (segment (start 61.74 59.1) (end 61.74 60.2253) (width 0.25) (layer B.Cu) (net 3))
 (via (at 60.4588 70.3) (size 0.8) (layers F.Cu B.Cu) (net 3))
 (via (at 61.9006 63.635) (size 0.8) (layers F.Cu B.Cu) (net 3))
 (segment (start 57.7854 66.2538) (end 57.1182 65.5866) (width 0.25) (layer F.Cu) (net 6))
 (segment (start 57.1182 65.5866) (end 57.0384 65.5866) (width 0.25) (layer F.Cu) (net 6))
 (segment (start 57.0384 65.5866) (end 56.7997 65.3479) (width 0.25) (layer F.Cu) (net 6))
 (segment (start 56.7997 65.3479) (end 56.7997 63.635) (width 0.25) (layer F.Cu) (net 6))
 (segment (start 61.93 70.3) (end 59.9137 68.2837) (width 0.25) (layer F.Cu) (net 6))
 (segment (start 59.9137 68.2837) (end 59.1411 68.2837) (width 0.25) (layer F.Cu) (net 6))
 (segment (start 59.1411 68.2837) (end 57.7854 66.928) (width 0.25) (layer F.Cu) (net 6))
 (segment (start 57.7854 66.928) (end 57.7854 66.2538) (width 0.25) (layer F.Cu) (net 6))
 (segment (start 57.7854 66.2538) (end 58.4702 65.569) (width 0.25) (layer F.Cu) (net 6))
 (segment (start 58.4702 65.569) (end 60.589 65.569) (width 0.25) (layer F.Cu) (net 6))
 (segment (start 60.589 65.569) (end 61.74 66.72) (width 0.25) (layer F.Cu) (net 6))
 (segment (start 57.9 63.635) (end 56.7997 63.635) (width 0.25) (layer F.Cu) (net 6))
 (segment (start 60.34 54.64) (end 60.34 55.8153) (width 0.25) (layer B.Cu) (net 6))
 (segment (start 61.74 65.5947) (end 60.5932 64.4479) (width 0.25) (layer B.Cu) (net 6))
 (segment (start 60.5932 64.4479) (end 60.5932 56.0685) (width 0.25) (layer B.Cu) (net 6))
 (segment (start 60.5932 56.0685) (end 60.34 55.8153) (width 0.25) (layer B.Cu) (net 6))
 (segment (start 61.74 66.72) (end 61.74 65.5947) (width 0.25) (layer B.Cu) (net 6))
 (segment (start 59.2 66.72) (end 60.3253 66.72) (width 0.25) (layer F.Cu) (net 4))
 (segment (start 64.47 70.3) (end 64.47 68.9026) (width 0.25) (layer F.Cu) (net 4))
 (segment (start 64.47 68.9026) (end 63.4127 67.8453) (width 0.25) (layer F.Cu) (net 4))
 (segment (start 63.4127 67.8453) (end 61.1692 67.8453) (width 0.25) (layer F.Cu) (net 4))
 (segment (start 61.1692 67.8453) (end 60.3253 67.0014) (width 0.25) (layer F.Cu) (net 4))
 (segment (start 60.3253 67.0014) (end 60.3253 66.72) (width 0.25) (layer F.Cu) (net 4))
 (segment (start 59.0003 62.365) (end 59.0003 62.8111) (width 0.25) (layer F.Cu) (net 4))
 (segment (start 59.0003 62.8111) (end 59.1947 63.0055) (width 0.25) (layer F.Cu) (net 4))
 (segment (start 59.2 65.5947) (end 59.2 63.0108) (width 0.25) (layer B.Cu) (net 4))
 (segment (start 59.2 63.0108) (end 59.1947 63.0055) (width 0.25) (layer B.Cu) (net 4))
 (segment (start 57.9 62.365) (end 59.0003 62.365) (width 0.25) (layer F.Cu) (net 4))
 (segment (start 59.2 66.72) (end 59.2 65.5947) (width 0.25) (layer B.Cu) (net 4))
 (via (at 59.1947 63.0055) (size 0.8) (layers F.Cu B.Cu) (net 4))
 (segment (start 67.31 58.166) (end 66.3347 58.166) (width 0.25) (layer F.Cu) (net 9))
 (segment (start 62.88 52.1) (end 62.88 53.2753) (width 0.25) (layer F.Cu) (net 9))
 (segment (start 62.88 53.2753) (end 63.2474 53.2753) (width 0.25) (layer F.Cu) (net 9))
 (segment (start 63.2474 53.2753) (end 64.0553 54.0832) (width 0.25) (layer F.Cu) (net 9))
 (segment (start 64.0553 54.0832) (end 64.0553 55.8866) (width 0.25) (layer F.Cu) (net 9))
 (segment (start 64.0553 55.8866) (end 66.3347 58.166) (width 0.25) (layer F.Cu) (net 9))
 (segment (start 68.2604 61.9839) (end 68.2604 65.2317) (width 0.25) (layer F.Cu) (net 5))
 (segment (start 68.2604 65.2317) (end 68.1478 65.3443) (width 0.25) (layer F.Cu) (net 5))
 (segment (start 68.1478 65.3443) (end 66.4795 65.3443) (width 0.25) (layer F.Cu) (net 5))
 (segment (start 66.4795 65.3443) (end 65.5474 64.4122) (width 0.25) (layer F.Cu) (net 5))
 (segment (start 65.5474 64.4122) (end 65.5474 63.5121) (width 0.25) (layer F.Cu) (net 5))
 (segment (start 65.5474 63.5121) (end 64.4003 62.365) (width 0.25) (layer F.Cu) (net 5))
 (segment (start 60.3253 59.1) (end 60.3253 59.3814) (width 0.25) (layer F.Cu) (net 5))
 (segment (start 60.3253 59.3814) (end 61.1692 60.2253) (width 0.25) (layer F.Cu) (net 5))
 (segment (start 61.1692 60.2253) (end 64.7106 60.2253) (width 0.25) (layer F.Cu) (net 5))
 (segment (start 64.7106 60.2253) (end 66.4692 61.9839) (width 0.25) (layer F.Cu) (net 5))
 (segment (start 66.4692 61.9839) (end 68.2604 61.9839) (width 0.25) (layer F.Cu) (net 5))
 (segment (start 72.2547 62.35) (end 72.2547 61.9701) (width 0.25) (layer F.Cu) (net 5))
 (segment (start 72.2547 61.9701) (end 71.5082 61.2236) (width 0.25) (layer F.Cu) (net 5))
 (segment (start 71.5082 61.2236) (end 69.0207 61.2236) (width 0.25) (layer F.Cu) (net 5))
 (segment (start 69.0207 61.2236) (end 68.2604 61.9839) (width 0.25) (layer F.Cu) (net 5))
 (segment (start 63.3 62.365) (end 64.4003 62.365) (width 0.25) (layer F.Cu) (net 5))
 (segment (start 59.2 59.1) (end 60.3253 59.1) (width 0.25) (layer F.Cu) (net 5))
 (segment (start 73.23 62.35) (end 72.2547 62.35) (width 0.25) (layer F.Cu) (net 5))
 (segment (start 64.28 59.1) (end 64.28 60.2253) (width 0.25) (layer B.Cu) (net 1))
 (segment (start 63.3 64.905) (end 64.4003 64.905) (width 0.25) (layer F.Cu) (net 1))
 (segment (start 64.8221 64.3703) (end 64.8221 60.7674) (width 0.25) (layer B.Cu) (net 1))
 (segment (start 64.8221 60.7674) (end 64.28 60.2253) (width 0.25) (layer B.Cu) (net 1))
 (segment (start 64.4003 64.905) (end 64.4003 64.7921) (width 0.25) (layer F.Cu) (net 1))
 (segment (start 64.4003 64.7921) (end 64.8221 64.3703) (width 0.25) (layer F.Cu) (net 1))
 (segment (start 64.28 59.1) (end 65.4053 59.1) (width 0.25) (layer F.Cu) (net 1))
 (segment (start 67.31 60.866) (end 66.3347 60.866) (width 0.25) (layer F.Cu) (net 1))
 (segment (start 66.3347 60.866) (end 65.4053 59.9366) (width 0.25) (layer F.Cu) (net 1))
 (segment (start 65.4053 59.9366) (end 65.4053 59.1) (width 0.25) (layer F.Cu) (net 1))
 (via (at 64.8221 64.3703) (size 0.8) (layers F.Cu B.Cu) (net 1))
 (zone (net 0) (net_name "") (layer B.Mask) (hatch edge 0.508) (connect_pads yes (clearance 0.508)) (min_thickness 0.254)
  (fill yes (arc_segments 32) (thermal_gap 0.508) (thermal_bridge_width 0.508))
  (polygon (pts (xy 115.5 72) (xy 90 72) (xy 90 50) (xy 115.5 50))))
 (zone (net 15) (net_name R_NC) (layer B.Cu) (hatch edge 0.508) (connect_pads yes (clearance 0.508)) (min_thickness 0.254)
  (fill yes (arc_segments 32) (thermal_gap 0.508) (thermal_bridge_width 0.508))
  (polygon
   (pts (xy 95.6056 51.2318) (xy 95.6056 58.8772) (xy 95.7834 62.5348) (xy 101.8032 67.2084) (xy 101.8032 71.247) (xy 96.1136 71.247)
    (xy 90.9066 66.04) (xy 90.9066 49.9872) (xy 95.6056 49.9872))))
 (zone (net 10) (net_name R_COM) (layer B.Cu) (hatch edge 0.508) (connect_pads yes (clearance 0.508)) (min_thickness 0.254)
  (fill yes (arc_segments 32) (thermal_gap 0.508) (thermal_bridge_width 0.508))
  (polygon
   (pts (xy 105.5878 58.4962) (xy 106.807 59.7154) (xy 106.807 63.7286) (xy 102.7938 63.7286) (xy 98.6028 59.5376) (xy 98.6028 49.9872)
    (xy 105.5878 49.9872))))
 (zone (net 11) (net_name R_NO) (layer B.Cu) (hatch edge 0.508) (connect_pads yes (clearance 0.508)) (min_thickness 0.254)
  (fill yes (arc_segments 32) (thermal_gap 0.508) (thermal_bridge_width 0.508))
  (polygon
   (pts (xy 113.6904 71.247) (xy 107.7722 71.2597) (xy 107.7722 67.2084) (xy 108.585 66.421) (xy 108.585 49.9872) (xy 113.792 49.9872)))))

